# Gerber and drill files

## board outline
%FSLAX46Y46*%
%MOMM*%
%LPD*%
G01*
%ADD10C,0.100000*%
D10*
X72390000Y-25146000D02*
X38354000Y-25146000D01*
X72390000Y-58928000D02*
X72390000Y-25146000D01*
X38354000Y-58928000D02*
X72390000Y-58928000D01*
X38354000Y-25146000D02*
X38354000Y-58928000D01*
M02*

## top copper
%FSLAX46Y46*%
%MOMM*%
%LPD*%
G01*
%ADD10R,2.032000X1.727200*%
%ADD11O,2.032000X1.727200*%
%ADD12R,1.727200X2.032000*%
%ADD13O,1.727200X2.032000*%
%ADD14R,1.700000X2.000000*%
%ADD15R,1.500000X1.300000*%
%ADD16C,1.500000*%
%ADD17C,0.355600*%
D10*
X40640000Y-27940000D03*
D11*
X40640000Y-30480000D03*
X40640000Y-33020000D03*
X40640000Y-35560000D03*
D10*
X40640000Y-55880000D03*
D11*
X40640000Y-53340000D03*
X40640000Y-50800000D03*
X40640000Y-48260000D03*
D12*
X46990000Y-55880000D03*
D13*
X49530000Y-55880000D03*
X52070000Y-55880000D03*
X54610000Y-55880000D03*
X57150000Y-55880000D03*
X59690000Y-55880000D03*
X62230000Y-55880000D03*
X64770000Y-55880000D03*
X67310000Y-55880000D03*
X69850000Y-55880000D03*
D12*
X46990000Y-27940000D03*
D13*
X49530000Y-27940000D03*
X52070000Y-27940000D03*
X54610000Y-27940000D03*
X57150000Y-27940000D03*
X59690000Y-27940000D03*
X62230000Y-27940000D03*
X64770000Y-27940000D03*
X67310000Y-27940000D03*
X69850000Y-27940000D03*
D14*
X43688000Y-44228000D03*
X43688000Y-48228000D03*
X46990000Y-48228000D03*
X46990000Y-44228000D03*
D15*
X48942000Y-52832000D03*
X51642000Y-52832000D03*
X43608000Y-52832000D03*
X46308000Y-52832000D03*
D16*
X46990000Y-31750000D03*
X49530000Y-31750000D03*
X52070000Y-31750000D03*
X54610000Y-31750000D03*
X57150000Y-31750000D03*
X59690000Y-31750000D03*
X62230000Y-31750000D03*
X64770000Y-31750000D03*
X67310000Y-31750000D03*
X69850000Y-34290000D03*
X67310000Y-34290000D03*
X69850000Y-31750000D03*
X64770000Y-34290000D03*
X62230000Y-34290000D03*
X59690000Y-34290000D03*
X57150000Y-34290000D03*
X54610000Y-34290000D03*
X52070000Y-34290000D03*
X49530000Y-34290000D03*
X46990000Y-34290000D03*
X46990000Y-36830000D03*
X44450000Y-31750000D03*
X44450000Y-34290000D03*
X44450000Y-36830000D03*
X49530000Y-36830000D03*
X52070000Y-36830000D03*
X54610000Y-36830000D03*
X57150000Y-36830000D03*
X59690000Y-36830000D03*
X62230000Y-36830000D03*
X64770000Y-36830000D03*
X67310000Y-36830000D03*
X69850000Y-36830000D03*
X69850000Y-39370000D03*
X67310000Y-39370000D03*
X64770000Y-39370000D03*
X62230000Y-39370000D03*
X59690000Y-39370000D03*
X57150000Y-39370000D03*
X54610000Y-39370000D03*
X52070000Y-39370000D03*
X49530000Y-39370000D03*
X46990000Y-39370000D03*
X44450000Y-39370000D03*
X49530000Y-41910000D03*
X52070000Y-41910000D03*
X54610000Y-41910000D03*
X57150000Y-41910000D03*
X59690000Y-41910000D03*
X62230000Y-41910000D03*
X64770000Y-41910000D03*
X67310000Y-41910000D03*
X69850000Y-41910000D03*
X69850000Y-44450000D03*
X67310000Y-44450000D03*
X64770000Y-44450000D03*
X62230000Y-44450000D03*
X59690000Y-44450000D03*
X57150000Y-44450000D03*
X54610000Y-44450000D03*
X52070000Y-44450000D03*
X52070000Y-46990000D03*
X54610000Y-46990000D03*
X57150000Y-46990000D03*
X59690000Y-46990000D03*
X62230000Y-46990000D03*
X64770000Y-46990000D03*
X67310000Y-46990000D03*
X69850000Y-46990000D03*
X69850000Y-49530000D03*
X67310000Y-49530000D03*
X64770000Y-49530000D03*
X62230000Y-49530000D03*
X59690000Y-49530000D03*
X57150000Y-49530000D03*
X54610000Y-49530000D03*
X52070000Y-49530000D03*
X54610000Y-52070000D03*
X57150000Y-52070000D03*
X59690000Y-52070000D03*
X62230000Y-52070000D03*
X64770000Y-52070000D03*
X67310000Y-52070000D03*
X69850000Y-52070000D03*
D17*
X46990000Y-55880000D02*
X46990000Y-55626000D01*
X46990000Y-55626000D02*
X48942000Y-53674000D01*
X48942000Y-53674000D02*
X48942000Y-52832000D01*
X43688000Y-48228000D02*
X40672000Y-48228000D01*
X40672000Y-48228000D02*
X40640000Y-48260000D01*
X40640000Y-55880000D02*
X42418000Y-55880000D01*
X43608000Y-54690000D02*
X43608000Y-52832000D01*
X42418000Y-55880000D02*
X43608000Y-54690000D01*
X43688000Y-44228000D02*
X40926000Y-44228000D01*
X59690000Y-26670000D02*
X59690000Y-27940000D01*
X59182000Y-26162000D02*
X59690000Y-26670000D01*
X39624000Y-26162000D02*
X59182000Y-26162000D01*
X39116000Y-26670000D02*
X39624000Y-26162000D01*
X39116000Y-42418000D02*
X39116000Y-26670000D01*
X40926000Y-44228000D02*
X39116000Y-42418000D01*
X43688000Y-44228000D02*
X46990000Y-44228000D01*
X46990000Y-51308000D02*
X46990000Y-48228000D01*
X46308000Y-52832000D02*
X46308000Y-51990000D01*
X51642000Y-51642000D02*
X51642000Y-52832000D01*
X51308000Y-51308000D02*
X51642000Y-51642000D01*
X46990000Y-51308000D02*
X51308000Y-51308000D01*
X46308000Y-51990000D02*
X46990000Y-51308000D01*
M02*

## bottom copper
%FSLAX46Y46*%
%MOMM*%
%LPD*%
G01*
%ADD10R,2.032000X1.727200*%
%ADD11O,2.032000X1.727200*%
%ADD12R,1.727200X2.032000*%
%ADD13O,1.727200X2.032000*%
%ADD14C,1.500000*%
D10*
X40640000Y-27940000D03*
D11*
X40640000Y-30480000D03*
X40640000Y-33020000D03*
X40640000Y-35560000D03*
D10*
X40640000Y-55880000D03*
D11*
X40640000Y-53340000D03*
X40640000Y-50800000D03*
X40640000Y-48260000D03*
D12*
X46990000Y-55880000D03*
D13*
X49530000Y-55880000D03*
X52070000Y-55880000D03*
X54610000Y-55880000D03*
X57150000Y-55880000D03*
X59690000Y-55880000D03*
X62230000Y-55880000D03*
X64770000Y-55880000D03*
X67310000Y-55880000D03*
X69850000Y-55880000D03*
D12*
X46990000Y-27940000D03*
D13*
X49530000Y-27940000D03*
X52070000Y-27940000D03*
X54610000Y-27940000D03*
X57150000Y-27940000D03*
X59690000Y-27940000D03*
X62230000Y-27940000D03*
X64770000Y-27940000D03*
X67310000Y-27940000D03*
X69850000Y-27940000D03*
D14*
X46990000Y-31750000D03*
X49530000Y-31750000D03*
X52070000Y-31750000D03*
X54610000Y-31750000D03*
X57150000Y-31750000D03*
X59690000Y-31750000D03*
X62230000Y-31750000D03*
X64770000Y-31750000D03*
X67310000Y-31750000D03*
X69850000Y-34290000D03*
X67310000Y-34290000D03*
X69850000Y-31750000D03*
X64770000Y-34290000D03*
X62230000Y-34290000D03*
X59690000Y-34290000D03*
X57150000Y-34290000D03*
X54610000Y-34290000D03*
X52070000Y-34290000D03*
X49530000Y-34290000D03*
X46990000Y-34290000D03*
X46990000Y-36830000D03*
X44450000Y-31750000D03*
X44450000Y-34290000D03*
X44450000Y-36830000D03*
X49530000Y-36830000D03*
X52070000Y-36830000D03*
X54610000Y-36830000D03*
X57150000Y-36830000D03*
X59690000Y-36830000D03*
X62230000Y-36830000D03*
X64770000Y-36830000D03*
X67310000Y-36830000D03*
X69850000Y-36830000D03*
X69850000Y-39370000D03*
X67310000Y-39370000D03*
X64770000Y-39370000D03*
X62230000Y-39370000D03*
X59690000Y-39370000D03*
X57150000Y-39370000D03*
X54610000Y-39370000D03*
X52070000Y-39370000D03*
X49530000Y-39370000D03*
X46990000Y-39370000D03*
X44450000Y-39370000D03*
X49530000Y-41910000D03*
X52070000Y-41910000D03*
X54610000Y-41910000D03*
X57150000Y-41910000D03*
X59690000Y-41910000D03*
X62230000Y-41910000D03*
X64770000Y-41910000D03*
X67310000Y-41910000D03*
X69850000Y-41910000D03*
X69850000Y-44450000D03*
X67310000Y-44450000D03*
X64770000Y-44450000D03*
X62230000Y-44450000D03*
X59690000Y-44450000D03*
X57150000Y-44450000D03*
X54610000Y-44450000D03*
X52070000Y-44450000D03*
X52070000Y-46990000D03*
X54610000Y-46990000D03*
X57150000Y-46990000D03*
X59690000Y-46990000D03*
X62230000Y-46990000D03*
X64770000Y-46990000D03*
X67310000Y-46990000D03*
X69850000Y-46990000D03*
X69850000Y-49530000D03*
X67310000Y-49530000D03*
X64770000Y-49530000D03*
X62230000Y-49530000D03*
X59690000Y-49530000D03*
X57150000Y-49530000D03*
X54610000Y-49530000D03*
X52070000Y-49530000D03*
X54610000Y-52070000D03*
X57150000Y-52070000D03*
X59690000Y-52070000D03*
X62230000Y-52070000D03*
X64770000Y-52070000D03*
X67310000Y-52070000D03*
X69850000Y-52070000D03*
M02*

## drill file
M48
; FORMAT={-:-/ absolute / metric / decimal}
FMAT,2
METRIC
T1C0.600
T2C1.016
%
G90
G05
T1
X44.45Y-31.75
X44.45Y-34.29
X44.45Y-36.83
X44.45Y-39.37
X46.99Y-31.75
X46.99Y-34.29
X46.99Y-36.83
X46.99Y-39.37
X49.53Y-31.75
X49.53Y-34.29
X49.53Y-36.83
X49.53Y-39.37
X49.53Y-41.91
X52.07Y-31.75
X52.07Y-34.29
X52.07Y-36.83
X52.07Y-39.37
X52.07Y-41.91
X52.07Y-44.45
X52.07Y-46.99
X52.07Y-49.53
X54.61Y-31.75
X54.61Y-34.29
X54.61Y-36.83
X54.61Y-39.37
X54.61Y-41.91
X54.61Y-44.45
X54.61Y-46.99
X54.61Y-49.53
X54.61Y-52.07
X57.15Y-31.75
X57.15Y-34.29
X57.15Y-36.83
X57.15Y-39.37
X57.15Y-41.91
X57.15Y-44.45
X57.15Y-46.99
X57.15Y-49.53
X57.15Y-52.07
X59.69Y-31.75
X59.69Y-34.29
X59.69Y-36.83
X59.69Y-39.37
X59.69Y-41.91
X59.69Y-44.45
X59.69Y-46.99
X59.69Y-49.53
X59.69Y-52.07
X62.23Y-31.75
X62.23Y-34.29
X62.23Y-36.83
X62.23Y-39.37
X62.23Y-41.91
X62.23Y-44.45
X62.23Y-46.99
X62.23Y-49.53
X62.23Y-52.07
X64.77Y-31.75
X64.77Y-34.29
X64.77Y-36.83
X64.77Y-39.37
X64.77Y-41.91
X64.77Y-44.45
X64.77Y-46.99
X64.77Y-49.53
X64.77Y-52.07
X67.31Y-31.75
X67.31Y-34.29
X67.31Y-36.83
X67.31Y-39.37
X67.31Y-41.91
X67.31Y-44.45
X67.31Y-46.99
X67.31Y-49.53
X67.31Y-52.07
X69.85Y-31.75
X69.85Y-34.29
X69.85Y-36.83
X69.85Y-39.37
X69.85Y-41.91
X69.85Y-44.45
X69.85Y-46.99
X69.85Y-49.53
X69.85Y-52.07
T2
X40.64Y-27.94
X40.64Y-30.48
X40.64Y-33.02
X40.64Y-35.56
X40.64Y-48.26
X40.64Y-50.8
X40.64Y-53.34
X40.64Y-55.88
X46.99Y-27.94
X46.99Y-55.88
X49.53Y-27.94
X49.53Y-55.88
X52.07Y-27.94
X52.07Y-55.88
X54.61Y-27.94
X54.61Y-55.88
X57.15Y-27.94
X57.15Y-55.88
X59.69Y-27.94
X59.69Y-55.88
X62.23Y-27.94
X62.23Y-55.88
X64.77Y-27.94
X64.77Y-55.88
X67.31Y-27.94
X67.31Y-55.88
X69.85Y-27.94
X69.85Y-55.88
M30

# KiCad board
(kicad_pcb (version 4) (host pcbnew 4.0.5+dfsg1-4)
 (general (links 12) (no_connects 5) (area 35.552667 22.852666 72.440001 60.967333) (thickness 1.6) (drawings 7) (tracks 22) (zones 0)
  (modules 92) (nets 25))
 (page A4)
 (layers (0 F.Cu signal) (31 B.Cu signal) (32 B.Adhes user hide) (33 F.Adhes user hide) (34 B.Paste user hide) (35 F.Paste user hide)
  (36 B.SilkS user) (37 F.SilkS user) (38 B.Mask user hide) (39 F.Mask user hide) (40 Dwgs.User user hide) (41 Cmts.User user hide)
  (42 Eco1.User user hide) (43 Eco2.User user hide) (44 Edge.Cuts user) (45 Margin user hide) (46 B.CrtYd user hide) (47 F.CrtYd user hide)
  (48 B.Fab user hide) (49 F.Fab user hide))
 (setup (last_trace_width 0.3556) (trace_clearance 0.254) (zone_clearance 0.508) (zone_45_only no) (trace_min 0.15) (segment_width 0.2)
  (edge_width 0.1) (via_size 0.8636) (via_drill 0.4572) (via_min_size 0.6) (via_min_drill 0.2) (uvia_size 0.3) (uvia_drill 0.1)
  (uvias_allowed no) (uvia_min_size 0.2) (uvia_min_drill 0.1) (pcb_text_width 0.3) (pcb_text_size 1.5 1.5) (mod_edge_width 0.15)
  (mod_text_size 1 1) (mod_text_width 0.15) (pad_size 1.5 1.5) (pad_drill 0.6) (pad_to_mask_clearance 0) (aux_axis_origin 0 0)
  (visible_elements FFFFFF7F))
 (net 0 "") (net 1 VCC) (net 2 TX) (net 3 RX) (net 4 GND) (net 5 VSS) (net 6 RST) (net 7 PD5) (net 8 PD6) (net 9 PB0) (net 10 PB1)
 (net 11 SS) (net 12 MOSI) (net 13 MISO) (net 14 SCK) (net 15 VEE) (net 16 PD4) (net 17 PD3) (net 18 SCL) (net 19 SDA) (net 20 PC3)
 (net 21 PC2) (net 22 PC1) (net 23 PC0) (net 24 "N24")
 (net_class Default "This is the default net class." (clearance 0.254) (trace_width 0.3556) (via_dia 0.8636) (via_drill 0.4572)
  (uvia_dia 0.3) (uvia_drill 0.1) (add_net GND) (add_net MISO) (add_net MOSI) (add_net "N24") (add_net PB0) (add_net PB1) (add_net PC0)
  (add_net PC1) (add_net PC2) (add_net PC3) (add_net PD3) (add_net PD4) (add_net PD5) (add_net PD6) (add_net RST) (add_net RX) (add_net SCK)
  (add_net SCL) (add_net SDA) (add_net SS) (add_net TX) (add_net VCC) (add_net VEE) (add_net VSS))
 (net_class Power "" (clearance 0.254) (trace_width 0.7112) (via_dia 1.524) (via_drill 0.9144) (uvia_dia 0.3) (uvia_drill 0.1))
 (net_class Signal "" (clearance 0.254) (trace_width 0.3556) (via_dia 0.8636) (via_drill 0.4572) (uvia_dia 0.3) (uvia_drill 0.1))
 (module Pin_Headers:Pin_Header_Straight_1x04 (layer F.Cu) (at 40.64 27.94)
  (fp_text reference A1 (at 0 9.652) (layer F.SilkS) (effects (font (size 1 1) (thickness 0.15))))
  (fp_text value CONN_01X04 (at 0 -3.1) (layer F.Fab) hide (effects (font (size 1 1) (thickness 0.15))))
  (pad 1 thru_hole rect (at 0 0) (size 2.032 1.7272) (drill 1.016) (layers *.Cu *.Mask) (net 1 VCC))
  (pad 2 thru_hole oval (at 0 2.54) (size 2.032 1.7272) (drill 1.016) (layers *.Cu *.Mask) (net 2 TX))
  (pad 3 thru_hole oval (at 0 5.08) (size 2.032 1.7272) (drill 1.016) (layers *.Cu *.Mask) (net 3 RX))
  (pad 4 thru_hole oval (at 0 7.62) (size 2.032 1.7272) (drill 1.016) (layers *.Cu *.Mask) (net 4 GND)))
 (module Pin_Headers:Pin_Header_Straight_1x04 (layer F.Cu) (at 40.64 55.88 180)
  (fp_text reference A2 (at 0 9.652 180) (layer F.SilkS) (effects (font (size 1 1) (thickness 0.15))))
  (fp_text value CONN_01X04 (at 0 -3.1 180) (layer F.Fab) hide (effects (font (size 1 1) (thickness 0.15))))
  (pad 1 thru_hole rect (at 0 0 180) (size 2.032 1.7272) (drill 1.016) (layers *.Cu *.Mask) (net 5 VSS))
  (pad 2 thru_hole oval (at 0 2.54 180) (size 2.032 1.7272) (drill 1.016) (layers *.Cu *.Mask) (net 1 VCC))
  (pad 3 thru_hole oval (at 0 5.08 180) (size 2.032 1.7272) (drill 1.016) (layers *.Cu *.Mask) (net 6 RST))
  (pad 4 thru_hole oval (at 0 7.62 180) (size 2.032 1.7272) (drill 1.016) (layers *.Cu *.Mask) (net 4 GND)))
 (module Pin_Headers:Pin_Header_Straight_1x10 (layer F.Cu) (at 46.99 55.88 90)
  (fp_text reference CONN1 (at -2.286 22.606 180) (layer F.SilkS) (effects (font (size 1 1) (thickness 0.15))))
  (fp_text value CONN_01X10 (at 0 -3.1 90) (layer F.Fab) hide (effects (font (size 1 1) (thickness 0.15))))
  (pad 1 thru_hole rect (at 0 0 90) (size 2.032 1.7272) (drill 1.016) (layers *.Cu *.Mask) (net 1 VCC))
  (pad 2 thru_hole oval (at 0 2.54 90) (size 2.032 1.7272) (drill 1.016) (layers *.Cu *.Mask) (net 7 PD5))
  (pad 3 thru_hole oval (at 0 5.08 90) (size 2.032 1.7272) (drill 1.016) (layers *.Cu *.Mask) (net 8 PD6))
  (pad 4 thru_hole oval (at 0 7.62 90) (size 2.032 1.7272) (drill 1.016) (layers *.Cu *.Mask) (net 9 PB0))
  (pad 5 thru_hole oval (at 0 10.16 90) (size 2.032 1.7272) (drill 1.016) (layers *.Cu *.Mask) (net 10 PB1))
  (pad 6 thru_hole oval (at 0 12.7 90) (size 2.032 1.7272) (drill 1.016) (layers *.Cu *.Mask) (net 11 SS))
  (pad 7 thru_hole oval (at 0 15.24 90) (size 2.032 1.7272) (drill 1.016) (layers *.Cu *.Mask) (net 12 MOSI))
  (pad 8 thru_hole oval (at 0 17.78 90) (size 2.032 1.7272) (drill 1.016) (layers *.Cu *.Mask) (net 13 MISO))
  (pad 9 thru_hole oval (at 0 20.32 90) (size 2.032 1.7272) (drill 1.016) (layers *.Cu *.Mask) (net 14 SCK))
  (pad 10 thru_hole oval (at 0 22.86 90) (size 2.032 1.7272) (drill 1.016) (layers *.Cu *.Mask) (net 4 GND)))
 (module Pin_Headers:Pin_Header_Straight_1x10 (layer F.Cu) (at 46.99 27.94 90)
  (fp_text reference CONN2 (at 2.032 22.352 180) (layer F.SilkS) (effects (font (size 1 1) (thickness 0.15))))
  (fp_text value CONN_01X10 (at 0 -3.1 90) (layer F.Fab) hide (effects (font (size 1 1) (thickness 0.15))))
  (pad 1 thru_hole rect (at 0 0 90) (size 2.032 1.7272) (drill 1.016) (layers *.Cu *.Mask) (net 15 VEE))
  (pad 2 thru_hole oval (at 0 2.54 90) (size 2.032 1.7272) (drill 1.016) (layers *.Cu *.Mask) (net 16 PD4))
  (pad 3 thru_hole oval (at 0 5.08 90) (size 2.032 1.7272) (drill 1.016) (layers *.Cu *.Mask) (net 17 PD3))
  (pad 4 thru_hole oval (at 0 7.62 90) (size 2.032 1.7272) (drill 1.016) (layers *.Cu *.Mask) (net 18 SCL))
  (pad 5 thru_hole oval (at 0 10.16 90) (size 2.032 1.7272) (drill 1.016) (layers *.Cu *.Mask) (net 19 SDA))
  (pad 6 thru_hole oval (at 0 12.7 90) (size 2.032 1.7272) (drill 1.016) (layers *.Cu *.Mask) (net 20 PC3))
  (pad 7 thru_hole oval (at 0 15.24 90) (size 2.032 1.7272) (drill 1.016) (layers *.Cu *.Mask) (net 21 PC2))
  (pad 8 thru_hole oval (at 0 17.78 90) (size 2.032 1.7272) (drill 1.016) (layers *.Cu *.Mask) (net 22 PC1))
  (pad 9 thru_hole oval (at 0 20.32 90) (size 2.032 1.7272) (drill 1.016) (layers *.Cu *.Mask) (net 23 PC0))
  (pad 10 thru_hole oval (at 0 22.86 90) (size 2.032 1.7272) (drill 1.016) (layers *.Cu *.Mask) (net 4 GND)))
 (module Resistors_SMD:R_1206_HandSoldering (layer F.Cu) (at 43.688 46.228 270)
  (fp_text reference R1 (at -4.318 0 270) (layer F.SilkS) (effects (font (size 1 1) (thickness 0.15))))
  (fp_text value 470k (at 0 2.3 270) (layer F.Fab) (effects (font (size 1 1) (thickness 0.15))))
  (pad 1 smd rect (at -2 0 270) (size 2 1.7) (layers F.Cu F.Paste F.Mask) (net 20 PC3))
  (pad 2 smd rect (at 2 0 270) (size 2 1.7) (layers F.Cu F.Paste F.Mask) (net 4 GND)))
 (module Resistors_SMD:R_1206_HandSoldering (layer F.Cu) (at 46.99 46.228 90)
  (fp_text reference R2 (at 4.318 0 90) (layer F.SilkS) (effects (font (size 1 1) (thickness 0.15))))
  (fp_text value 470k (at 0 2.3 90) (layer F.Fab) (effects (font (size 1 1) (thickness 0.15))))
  (pad 1 smd rect (at -2 0 90) (size 2 1.7) (layers F.Cu F.Paste F.Mask) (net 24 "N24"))
  (pad 2 smd rect (at 2 0 90) (size 2 1.7) (layers F.Cu F.Paste F.Mask) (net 20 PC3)))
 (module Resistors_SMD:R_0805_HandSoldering (layer F.Cu) (at 50.292 52.832)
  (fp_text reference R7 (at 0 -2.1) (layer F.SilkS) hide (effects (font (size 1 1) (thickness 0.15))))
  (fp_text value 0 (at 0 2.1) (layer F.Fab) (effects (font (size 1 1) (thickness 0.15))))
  (pad 1 smd rect (at -1.35 0) (size 1.5 1.3) (layers F.Cu F.Paste F.Mask) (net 1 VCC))
  (pad 2 smd rect (at 1.35 0) (size 1.5 1.3) (layers F.Cu F.Paste F.Mask) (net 24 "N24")))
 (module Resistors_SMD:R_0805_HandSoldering (layer F.Cu) (at 44.958 52.832)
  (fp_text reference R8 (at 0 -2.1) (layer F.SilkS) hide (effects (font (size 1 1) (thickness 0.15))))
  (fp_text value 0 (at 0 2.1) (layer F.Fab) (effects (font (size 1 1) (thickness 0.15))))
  (pad 1 smd rect (at -1.35 0) (size 1.5 1.3) (layers F.Cu F.Paste F.Mask) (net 5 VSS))
  (pad 2 smd rect (at 1.35 0) (size 1.5 1.3) (layers F.Cu F.Paste F.Mask) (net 24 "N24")))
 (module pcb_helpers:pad (layer F.Cu) (at 46.99 31.75)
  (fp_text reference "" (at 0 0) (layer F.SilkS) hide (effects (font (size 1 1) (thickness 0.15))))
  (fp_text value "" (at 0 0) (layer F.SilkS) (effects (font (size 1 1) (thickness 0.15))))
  (pad 1 thru_hole circle (at 0 0) (size 1.5 1.5) (drill 0.6) (layers *.Cu *.Mask F.SilkS)))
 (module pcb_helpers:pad (layer F.Cu) (at 49.53 31.75)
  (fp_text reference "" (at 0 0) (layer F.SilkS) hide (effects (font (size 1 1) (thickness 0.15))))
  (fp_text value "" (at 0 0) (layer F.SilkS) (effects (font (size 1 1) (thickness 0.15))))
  (pad 1 thru_hole circle (at 0 0) (size 1.5 1.5) (drill 0.6) (layers *.Cu *.Mask F.SilkS)))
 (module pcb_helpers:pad (layer F.Cu) (at 52.07 31.75)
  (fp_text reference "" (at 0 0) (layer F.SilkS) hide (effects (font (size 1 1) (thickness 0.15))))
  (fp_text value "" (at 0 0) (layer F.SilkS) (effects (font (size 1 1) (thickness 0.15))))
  (pad 1 thru_hole circle (at 0 0) (size 1.5 1.5) (drill 0.6) (layers *.Cu *.Mask F.SilkS)))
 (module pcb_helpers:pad (layer F.Cu) (at 54.61 31.75)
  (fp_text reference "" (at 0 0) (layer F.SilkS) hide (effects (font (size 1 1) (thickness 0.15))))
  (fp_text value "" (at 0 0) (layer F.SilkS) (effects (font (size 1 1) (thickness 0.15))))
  (pad 1 thru_hole circle (at 0 0) (size 1.5 1.5) (drill 0.6) (layers *.Cu *.Mask F.SilkS)))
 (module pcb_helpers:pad (layer F.Cu) (at 57.15 31.75)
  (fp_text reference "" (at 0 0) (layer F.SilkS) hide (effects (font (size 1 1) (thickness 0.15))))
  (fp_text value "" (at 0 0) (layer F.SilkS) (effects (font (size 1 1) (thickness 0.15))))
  (pad 1 thru_hole circle (at 0 0) (size 1.5 1.5) (drill 0.6) (layers *.Cu *.Mask F.SilkS)))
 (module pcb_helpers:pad (layer F.Cu) (at 59.69 31.75)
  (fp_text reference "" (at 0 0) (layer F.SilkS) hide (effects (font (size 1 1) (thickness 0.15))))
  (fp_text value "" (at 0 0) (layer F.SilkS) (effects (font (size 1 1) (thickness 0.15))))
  (pad 1 thru_hole circle (at 0 0) (size 1.5 1.5) (drill 0.6) (layers *.Cu *.Mask F.SilkS)))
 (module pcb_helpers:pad (layer F.Cu) (at 62.23 31.75)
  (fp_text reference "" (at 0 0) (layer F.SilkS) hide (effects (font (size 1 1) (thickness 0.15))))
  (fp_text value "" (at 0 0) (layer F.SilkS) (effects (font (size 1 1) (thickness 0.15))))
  (pad 1 thru_hole circle (at 0 0) (size 1.5 1.5) (drill 0.6) (layers *.Cu *.Mask F.SilkS)))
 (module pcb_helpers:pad (layer F.Cu) (at 64.77 31.75)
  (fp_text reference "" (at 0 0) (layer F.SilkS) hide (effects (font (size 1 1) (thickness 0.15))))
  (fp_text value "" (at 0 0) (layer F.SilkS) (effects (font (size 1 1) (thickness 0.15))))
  (pad 1 thru_hole circle (at 0 0) (size 1.5 1.5) (drill 0.6) (layers *.Cu *.Mask F.SilkS)))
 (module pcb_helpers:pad (layer F.Cu) (at 67.31 31.75)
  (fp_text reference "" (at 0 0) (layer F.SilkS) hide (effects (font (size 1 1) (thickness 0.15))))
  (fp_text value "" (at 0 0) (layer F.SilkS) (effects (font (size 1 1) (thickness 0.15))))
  (pad 1 thru_hole circle (at 0 0) (size 1.5 1.5) (drill 0.6) (layers *.Cu *.Mask F.SilkS)))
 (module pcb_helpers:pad (layer F.Cu) (at 69.85 34.29)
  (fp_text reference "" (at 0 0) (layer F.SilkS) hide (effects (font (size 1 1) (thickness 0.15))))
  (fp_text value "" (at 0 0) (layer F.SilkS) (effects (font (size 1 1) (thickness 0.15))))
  (pad 1 thru_hole circle (at 0 0) (size 1.5 1.5) (drill 0.6) (layers *.Cu *.Mask F.SilkS)))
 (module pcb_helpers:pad (layer F.Cu) (at 67.31 34.29)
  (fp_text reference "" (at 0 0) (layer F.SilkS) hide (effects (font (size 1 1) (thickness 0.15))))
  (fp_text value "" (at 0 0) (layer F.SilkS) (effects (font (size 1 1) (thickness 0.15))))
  (pad 1 thru_hole circle (at 0 0) (size 1.5 1.5) (drill 0.6) (layers *.Cu *.Mask F.SilkS)))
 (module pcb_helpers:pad (layer F.Cu) (at 69.85 31.75)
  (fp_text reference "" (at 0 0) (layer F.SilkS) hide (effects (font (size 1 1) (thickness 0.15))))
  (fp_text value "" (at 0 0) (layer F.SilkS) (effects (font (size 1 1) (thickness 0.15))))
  (pad 1 thru_hole circle (at 0 0) (size 1.5 1.5) (drill 0.6) (layers *.Cu *.Mask F.SilkS)))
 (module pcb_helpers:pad (layer F.Cu) (at 64.77 34.29)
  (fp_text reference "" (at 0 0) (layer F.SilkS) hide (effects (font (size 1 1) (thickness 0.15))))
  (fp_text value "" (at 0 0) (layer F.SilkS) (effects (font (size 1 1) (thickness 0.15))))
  (pad 1 thru_hole circle (at 0 0) (size 1.5 1.5) (drill 0.6) (layers *.Cu *.Mask F.SilkS)))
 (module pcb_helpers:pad (layer F.Cu) (at 62.23 34.29)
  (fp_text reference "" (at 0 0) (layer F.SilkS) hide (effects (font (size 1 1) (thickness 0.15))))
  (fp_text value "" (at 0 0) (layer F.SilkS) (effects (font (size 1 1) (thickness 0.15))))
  (pad 1 thru_hole circle (at 0 0) (size 1.5 1.5) (drill 0.6) (layers *.Cu *.Mask F.SilkS)))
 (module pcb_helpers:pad (layer F.Cu) (at 59.69 34.29)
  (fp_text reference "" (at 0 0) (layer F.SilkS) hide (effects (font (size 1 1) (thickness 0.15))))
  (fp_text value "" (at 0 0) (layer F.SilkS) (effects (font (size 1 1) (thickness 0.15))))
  (pad 1 thru_hole circle (at 0 0) (size 1.5 1.5) (drill 0.6) (layers *.Cu *.Mask F.SilkS)))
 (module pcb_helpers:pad (layer F.Cu) (at 57.15 34.29)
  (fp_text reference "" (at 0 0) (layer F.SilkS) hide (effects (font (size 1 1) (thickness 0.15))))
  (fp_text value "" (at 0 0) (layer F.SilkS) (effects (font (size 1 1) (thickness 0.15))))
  (pad 1 thru_hole circle (at 0 0) (size 1.5 1.5) (drill 0.6) (layers *.Cu *.Mask F.SilkS)))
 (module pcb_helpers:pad (layer F.Cu) (at 54.61 34.29)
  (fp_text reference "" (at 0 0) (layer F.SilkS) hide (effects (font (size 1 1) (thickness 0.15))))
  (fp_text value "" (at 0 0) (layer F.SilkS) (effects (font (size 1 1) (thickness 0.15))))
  (pad 1 thru_hole circle (at 0 0) (size 1.5 1.5) (drill 0.6) (layers *.Cu *.Mask F.SilkS)))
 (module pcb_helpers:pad (layer F.Cu) (at 52.07 34.29)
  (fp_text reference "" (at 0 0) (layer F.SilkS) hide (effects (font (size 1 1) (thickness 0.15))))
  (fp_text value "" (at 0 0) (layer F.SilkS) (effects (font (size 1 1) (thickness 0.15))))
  (pad 1 thru_hole circle (at 0 0) (size 1.5 1.5) (drill 0.6) (layers *.Cu *.Mask F.SilkS)))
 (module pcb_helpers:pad (layer F.Cu) (at 49.53 34.29)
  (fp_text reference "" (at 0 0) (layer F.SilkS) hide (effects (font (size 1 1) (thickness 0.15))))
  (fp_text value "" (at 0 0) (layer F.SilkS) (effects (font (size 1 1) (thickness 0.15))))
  (pad 1 thru_hole circle (at 0 0) (size 1.5 1.5) (drill 0.6) (layers *.Cu *.Mask F.SilkS)))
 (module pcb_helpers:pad (layer F.Cu) (at 46.99 34.29)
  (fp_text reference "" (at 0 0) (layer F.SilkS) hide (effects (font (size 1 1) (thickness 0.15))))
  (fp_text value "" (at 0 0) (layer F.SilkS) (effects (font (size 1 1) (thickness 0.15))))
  (pad 1 thru_hole circle (at 0 0) (size 1.5 1.5) (drill 0.6) (layers *.Cu *.Mask F.SilkS)))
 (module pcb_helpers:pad (layer F.Cu) (at 46.99 36.83)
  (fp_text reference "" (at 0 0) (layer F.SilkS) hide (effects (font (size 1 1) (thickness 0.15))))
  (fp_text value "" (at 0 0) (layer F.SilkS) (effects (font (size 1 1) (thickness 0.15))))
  (pad 1 thru_hole circle (at 0 0) (size 1.5 1.5) (drill 0.6) (layers *.Cu *.Mask F.SilkS)))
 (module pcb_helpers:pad (layer F.Cu) (at 44.45 31.75)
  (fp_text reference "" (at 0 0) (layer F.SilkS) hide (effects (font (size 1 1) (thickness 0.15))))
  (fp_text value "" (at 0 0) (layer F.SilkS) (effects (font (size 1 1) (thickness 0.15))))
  (pad 1 thru_hole circle (at 0 0) (size 1.5 1.5) (drill 0.6) (layers *.Cu *.Mask F.SilkS)))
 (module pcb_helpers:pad (layer F.Cu) (at 44.45 34.29)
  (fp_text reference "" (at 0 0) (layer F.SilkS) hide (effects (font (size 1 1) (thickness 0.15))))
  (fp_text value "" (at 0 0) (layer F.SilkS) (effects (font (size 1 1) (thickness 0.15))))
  (pad 1 thru_hole circle (at 0 0) (size 1.5 1.5) (drill 0.6) (layers *.Cu *.Mask F.SilkS)))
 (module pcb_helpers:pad (layer F.Cu) (at 44.45 36.83)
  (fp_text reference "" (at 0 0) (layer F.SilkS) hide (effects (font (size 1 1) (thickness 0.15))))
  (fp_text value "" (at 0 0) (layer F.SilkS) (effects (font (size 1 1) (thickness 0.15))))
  (pad 1 thru_hole circle (at 0 0) (size 1.5 1.5) (drill 0.6) (layers *.Cu *.Mask F.SilkS)))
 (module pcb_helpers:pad (layer F.Cu) (at 49.53 36.83)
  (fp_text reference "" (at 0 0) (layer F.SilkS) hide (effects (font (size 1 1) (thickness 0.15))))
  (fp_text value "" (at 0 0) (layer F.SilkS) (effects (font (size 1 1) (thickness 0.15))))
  (pad 1 thru_hole circle (at 0 0) (size 1.5 1.5) (drill 0.6) (layers *.Cu *.Mask F.SilkS)))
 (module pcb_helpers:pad (layer F.Cu) (at 52.07 36.83)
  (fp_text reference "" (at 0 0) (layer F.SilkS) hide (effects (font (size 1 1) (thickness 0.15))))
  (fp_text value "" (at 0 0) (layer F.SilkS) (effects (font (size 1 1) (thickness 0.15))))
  (pad 1 thru_hole circle (at 0 0) (size 1.5 1.5) (drill 0.6) (layers *.Cu *.Mask F.SilkS)))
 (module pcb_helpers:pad (layer F.Cu) (at 54.61 36.83)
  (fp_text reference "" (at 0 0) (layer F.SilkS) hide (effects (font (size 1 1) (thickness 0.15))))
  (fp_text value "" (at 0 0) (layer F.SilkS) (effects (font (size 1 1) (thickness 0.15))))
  (pad 1 thru_hole circle (at 0 0) (size 1.5 1.5) (drill 0.6) (layers *.Cu *.Mask F.SilkS)))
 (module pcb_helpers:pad (layer F.Cu) (at 57.15 36.83)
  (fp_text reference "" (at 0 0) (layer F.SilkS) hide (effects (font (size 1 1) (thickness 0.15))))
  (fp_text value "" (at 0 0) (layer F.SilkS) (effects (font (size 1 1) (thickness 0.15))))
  (pad 1 thru_hole circle (at 0 0) (size 1.5 1.5) (drill 0.6) (layers *.Cu *.Mask F.SilkS)))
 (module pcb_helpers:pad (layer F.Cu) (at 59.69 36.83)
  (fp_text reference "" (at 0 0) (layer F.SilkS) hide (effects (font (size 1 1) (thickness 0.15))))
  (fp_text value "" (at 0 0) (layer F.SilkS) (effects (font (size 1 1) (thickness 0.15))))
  (pad 1 thru_hole circle (at 0 0) (size 1.5 1.5) (drill 0.6) (layers *.Cu *.Mask F.SilkS)))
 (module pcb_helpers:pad (layer F.Cu) (at 62.23 36.83)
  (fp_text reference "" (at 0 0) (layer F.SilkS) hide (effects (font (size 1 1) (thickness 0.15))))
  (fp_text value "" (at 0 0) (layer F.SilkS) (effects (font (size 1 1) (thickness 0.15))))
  (pad 1 thru_hole circle (at 0 0) (size 1.5 1.5) (drill 0.6) (layers *.Cu *.Mask F.SilkS)))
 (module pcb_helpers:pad (layer F.Cu) (at 64.77 36.83)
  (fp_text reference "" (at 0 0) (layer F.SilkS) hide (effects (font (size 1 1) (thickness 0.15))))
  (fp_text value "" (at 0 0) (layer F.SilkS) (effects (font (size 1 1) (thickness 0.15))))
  (pad 1 thru_hole circle (at 0 0) (size 1.5 1.5) (drill 0.6) (layers *.Cu *.Mask F.SilkS)))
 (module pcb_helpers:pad (layer F.Cu) (at 67.31 36.83)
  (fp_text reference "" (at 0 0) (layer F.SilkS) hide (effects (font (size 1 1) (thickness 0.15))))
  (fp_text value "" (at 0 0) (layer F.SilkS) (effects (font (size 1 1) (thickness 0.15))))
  (pad 1 thru_hole circle (at 0 0) (size 1.5 1.5) (drill 0.6) (layers *.Cu *.Mask F.SilkS)))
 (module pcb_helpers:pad (layer F.Cu) (at 69.85 36.83)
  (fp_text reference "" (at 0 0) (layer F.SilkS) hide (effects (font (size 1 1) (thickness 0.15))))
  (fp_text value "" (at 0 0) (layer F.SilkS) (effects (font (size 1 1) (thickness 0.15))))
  (pad 1 thru_hole circle (at 0 0) (size 1.5 1.5) (drill 0.6) (layers *.Cu *.Mask F.SilkS)))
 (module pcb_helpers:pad (layer F.Cu) (at 69.85 39.37)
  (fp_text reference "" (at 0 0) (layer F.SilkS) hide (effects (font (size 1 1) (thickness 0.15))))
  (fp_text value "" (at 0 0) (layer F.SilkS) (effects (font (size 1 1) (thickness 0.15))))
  (pad 1 thru_hole circle (at 0 0) (size 1.5 1.5) (drill 0.6) (layers *.Cu *.Mask F.SilkS)))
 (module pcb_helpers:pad (layer F.Cu) (at 67.31 39.37)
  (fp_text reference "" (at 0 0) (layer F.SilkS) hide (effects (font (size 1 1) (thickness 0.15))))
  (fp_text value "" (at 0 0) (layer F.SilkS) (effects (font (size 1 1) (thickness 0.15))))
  (pad 1 thru_hole circle (at 0 0) (size 1.5 1.5) (drill 0.6) (layers *.Cu *.Mask F.SilkS)))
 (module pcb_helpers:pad (layer F.Cu) (at 64.77 39.37)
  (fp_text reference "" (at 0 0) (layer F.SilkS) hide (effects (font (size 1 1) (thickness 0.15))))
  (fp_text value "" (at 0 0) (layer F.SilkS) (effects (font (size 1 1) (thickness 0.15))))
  (pad 1 thru_hole circle (at 0 0) (size 1.5 1.5) (drill 0.6) (layers *.Cu *.Mask F.SilkS)))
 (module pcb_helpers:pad (layer F.Cu) (at 62.23 39.37)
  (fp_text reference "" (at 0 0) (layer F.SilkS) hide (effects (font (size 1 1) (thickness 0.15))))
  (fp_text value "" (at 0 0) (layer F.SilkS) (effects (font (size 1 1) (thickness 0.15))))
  (pad 1 thru_hole circle (at 0 0) (size 1.5 1.5) (drill 0.6) (layers *.Cu *.Mask F.SilkS)))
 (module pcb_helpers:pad (layer F.Cu) (at 59.69 39.37)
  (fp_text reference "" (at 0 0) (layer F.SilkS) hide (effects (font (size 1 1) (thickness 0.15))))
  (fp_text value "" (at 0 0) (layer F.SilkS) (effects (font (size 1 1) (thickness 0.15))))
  (pad 1 thru_hole circle (at 0 0) (size 1.5 1.5) (drill 0.6) (layers *.Cu *.Mask F.SilkS)))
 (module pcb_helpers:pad (layer F.Cu) (at 57.15 39.37)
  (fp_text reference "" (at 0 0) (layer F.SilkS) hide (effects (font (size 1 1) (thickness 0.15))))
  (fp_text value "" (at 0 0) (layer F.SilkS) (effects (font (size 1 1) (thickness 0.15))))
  (pad 1 thru_hole circle (at 0 0) (size 1.5 1.5) (drill 0.6) (layers *.Cu *.Mask F.SilkS)))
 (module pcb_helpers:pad (layer F.Cu) (at 54.61 39.37)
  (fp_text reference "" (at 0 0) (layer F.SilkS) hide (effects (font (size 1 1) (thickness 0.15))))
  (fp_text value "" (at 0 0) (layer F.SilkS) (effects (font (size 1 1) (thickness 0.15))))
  (pad 1 thru_hole circle (at 0 0) (size 1.5 1.5) (drill 0.6) (layers *.Cu *.Mask F.SilkS)))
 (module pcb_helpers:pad (layer F.Cu) (at 52.07 39.37)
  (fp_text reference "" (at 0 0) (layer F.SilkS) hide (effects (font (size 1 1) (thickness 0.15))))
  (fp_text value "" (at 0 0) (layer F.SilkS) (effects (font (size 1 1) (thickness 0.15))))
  (pad 1 thru_hole circle (at 0 0) (size 1.5 1.5) (drill 0.6) (layers *.Cu *.Mask F.SilkS)))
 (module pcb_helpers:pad (layer F.Cu) (at 49.53 39.37)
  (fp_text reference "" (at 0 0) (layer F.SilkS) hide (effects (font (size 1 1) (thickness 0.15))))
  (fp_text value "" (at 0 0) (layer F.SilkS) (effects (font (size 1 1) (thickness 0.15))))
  (pad 1 thru_hole circle (at 0 0) (size 1.5 1.5) (drill 0.6) (layers *.Cu *.Mask F.SilkS)))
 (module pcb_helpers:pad (layer F.Cu) (at 46.99 39.37)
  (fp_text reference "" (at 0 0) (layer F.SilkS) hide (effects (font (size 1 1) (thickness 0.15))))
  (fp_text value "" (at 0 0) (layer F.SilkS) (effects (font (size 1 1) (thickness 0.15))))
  (pad 1 thru_hole circle (at 0 0) (size 1.5 1.5) (drill 0.6) (layers *.Cu *.Mask F.SilkS)))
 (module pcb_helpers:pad (layer F.Cu) (at 44.45 39.37)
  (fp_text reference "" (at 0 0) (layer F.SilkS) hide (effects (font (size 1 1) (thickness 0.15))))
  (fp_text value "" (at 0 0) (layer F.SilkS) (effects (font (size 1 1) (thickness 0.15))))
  (pad 1 thru_hole circle (at 0 0) (size 1.5 1.5) (drill 0.6) (layers *.Cu *.Mask F.SilkS)))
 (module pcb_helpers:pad (layer F.Cu) (at 49.53 41.91)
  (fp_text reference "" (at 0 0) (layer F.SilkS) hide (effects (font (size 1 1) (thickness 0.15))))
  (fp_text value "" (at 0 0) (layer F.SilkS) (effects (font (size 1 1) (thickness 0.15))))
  (pad 1 thru_hole circle (at 0 0) (size 1.5 1.5) (drill 0.6) (layers *.Cu *.Mask F.SilkS)))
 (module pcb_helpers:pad (layer F.Cu) (at 52.07 41.91)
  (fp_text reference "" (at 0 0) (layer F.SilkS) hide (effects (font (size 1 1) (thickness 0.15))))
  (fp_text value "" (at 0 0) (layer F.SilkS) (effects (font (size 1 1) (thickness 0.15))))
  (pad 1 thru_hole circle (at 0 0) (size 1.5 1.5) (drill 0.6) (layers *.Cu *.Mask F.SilkS)))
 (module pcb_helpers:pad (layer F.Cu) (at 54.61 41.91)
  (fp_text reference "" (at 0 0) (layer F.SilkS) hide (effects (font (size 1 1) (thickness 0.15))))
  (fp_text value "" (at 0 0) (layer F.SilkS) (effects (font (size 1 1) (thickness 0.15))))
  (pad 1 thru_hole circle (at 0 0) (size 1.5 1.5) (drill 0.6) (layers *.Cu *.Mask F.SilkS)))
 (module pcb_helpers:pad (layer F.Cu) (at 57.15 41.91)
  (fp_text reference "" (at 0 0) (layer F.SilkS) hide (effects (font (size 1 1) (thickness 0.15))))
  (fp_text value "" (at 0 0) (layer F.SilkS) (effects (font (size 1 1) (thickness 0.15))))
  (pad 1 thru_hole circle (at 0 0) (size 1.5 1.5) (drill 0.6) (layers *.Cu *.Mask F.SilkS)))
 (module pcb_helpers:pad (layer F.Cu) (at 59.69 41.91)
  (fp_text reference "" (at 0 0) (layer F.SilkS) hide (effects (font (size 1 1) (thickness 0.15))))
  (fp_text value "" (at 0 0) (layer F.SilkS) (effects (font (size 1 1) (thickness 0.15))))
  (pad 1 thru_hole circle (at 0 0) (size 1.5 1.5) (drill 0.6) (layers *.Cu *.Mask F.SilkS)))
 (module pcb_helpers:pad (layer F.Cu) (at 62.23 41.91)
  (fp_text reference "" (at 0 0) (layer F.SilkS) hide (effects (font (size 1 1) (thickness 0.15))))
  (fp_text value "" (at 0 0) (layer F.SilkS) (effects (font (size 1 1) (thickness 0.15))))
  (pad 1 thru_hole circle (at 0 0) (size 1.5 1.5) (drill 0.6) (layers *.Cu *.Mask F.SilkS)))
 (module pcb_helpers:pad (layer F.Cu) (at 64.77 41.91)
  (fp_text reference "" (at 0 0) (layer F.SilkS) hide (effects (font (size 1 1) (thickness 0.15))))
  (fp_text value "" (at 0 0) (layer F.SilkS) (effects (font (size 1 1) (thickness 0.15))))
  (pad 1 thru_hole circle (at 0 0) (size 1.5 1.5) (drill 0.6) (layers *.Cu *.Mask F.SilkS)))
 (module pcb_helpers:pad (layer F.Cu) (at 67.31 41.91)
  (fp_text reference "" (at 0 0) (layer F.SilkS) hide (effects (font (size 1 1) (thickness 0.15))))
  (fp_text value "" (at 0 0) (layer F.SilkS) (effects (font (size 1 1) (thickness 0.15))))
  (pad 1 thru_hole circle (at 0 0) (size 1.5 1.5) (drill 0.6) (layers *.Cu *.Mask F.SilkS)))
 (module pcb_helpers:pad (layer F.Cu) (at 69.85 41.91)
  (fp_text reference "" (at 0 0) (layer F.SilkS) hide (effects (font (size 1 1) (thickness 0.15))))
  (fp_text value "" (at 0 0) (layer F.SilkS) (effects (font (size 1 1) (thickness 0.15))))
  (pad 1 thru_hole circle (at 0 0) (size 1.5 1.5) (drill 0.6) (layers *.Cu *.Mask F.SilkS)))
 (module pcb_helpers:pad (layer F.Cu) (at 69.85 44.45)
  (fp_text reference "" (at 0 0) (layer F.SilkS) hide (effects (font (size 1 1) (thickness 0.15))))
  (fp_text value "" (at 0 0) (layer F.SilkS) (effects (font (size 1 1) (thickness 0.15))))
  (pad 1 thru_hole circle (at 0 0) (size 1.5 1.5) (drill 0.6) (layers *.Cu *.Mask F.SilkS)))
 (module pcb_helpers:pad (layer F.Cu) (at 67.31 44.45)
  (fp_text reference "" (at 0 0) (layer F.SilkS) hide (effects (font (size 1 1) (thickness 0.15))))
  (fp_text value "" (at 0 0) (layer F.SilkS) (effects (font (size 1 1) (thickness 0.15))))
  (pad 1 thru_hole circle (at 0 0) (size 1.5 1.5) (drill 0.6) (layers *.Cu *.Mask F.SilkS)))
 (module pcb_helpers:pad (layer F.Cu) (at 64.77 44.45)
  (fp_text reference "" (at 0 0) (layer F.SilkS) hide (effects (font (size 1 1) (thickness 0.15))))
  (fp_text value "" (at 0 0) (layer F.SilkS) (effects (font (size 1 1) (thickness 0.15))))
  (pad 1 thru_hole circle (at 0 0) (size 1.5 1.5) (drill 0.6) (layers *.Cu *.Mask F.SilkS)))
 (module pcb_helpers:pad (layer F.Cu) (at 62.23 44.45)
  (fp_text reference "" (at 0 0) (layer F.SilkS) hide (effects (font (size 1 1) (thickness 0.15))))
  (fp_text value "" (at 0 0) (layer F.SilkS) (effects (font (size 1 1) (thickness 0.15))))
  (pad 1 thru_hole circle (at 0 0) (size 1.5 1.5) (drill 0.6) (layers *.Cu *.Mask F.SilkS)))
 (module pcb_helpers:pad (layer F.Cu) (at 59.69 44.45)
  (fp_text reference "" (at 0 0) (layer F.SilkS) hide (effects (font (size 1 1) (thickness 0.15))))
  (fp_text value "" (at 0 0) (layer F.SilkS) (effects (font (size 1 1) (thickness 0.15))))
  (pad 1 thru_hole circle (at 0 0) (size 1.5 1.5) (drill 0.6) (layers *.Cu *.Mask F.SilkS)))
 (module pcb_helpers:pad (layer F.Cu) (at 57.15 44.45)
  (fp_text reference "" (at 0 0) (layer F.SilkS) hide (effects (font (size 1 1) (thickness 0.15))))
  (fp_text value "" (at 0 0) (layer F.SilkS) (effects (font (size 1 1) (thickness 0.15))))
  (pad 1 thru_hole circle (at 0 0) (size 1.5 1.5) (drill 0.6) (layers *.Cu *.Mask F.SilkS)))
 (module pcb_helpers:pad (layer F.Cu) (at 54.61 44.45)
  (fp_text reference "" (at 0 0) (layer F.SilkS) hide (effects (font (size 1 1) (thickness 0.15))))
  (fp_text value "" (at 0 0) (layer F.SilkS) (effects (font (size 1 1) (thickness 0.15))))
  (pad 1 thru_hole circle (at 0 0) (size 1.5 1.5) (drill 0.6) (layers *.Cu *.Mask F.SilkS)))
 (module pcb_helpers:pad (layer F.Cu) (at 52.07 44.45)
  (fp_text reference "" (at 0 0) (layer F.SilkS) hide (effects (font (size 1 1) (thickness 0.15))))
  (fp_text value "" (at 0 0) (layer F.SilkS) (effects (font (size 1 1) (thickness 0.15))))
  (pad 1 thru_hole circle (at 0 0) (size 1.5 1.5) (drill 0.6) (layers *.Cu *.Mask F.SilkS)))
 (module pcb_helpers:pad (layer F.Cu) (at 52.07 46.99)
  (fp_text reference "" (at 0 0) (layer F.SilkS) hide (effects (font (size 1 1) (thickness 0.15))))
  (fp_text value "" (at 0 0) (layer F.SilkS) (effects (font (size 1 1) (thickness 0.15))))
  (pad 1 thru_hole circle (at 0 0) (size 1.5 1.5) (drill 0.6) (layers *.Cu *.Mask F.SilkS)))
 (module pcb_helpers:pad (layer F.Cu) (at 54.61 46.99)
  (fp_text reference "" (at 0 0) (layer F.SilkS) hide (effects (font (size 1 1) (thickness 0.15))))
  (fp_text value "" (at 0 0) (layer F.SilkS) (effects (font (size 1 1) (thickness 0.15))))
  (pad 1 thru_hole circle (at 0 0) (size 1.5 1.5) (drill 0.6) (layers *.Cu *.Mask F.SilkS)))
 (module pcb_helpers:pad (layer F.Cu) (at 57.15 46.99)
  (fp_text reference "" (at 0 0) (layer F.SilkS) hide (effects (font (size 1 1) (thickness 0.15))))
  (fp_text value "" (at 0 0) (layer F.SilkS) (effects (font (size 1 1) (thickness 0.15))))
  (pad 1 thru_hole circle (at 0 0) (size 1.5 1.5) (drill 0.6) (layers *.Cu *.Mask F.SilkS)))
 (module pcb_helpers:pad (layer F.Cu) (at 59.69 46.99)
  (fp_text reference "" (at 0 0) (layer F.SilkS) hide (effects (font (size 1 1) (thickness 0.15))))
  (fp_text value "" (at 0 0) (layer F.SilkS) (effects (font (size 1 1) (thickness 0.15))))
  (pad 1 thru_hole circle (at 0 0) (size 1.5 1.5) (drill 0.6) (layers *.Cu *.Mask F.SilkS)))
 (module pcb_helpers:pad (layer F.Cu) (at 62.23 46.99)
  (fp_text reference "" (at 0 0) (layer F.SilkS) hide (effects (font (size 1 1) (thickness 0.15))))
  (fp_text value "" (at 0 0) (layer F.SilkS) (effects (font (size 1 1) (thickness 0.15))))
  (pad 1 thru_hole circle (at 0 0) (size 1.5 1.5) (drill 0.6) (layers *.Cu *.Mask F.SilkS)))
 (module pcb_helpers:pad (layer F.Cu) (at 64.77 46.99)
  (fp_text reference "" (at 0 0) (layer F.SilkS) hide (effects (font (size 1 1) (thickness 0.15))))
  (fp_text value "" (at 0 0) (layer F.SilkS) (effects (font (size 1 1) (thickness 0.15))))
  (pad 1 thru_hole circle (at 0 0) (size 1.5 1.5) (drill 0.6) (layers *.Cu *.Mask F.SilkS)))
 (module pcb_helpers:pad (layer F.Cu) (at 67.31 46.99)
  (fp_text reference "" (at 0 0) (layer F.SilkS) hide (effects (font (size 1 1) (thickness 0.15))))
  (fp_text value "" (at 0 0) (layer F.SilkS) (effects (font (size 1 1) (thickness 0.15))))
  (pad 1 thru_hole circle (at 0 0) (size 1.5 1.5) (drill 0.6) (layers *.Cu *.Mask F.SilkS)))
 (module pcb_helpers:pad (layer F.Cu) (at 69.85 46.99)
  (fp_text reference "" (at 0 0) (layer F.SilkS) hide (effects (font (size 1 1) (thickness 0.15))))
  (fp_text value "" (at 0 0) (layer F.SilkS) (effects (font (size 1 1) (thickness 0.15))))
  (pad 1 thru_hole circle (at 0 0) (size 1.5 1.5) (drill 0.6) (layers *.Cu *.Mask F.SilkS)))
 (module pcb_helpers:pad (layer F.Cu) (at 69.85 49.53)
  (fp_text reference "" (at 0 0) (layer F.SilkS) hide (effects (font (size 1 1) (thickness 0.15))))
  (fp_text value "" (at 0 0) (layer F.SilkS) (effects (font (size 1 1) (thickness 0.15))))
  (pad 1 thru_hole circle (at 0 0) (size 1.5 1.5) (drill 0.6) (layers *.Cu *.Mask F.SilkS)))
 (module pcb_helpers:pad (layer F.Cu) (at 67.31 49.53)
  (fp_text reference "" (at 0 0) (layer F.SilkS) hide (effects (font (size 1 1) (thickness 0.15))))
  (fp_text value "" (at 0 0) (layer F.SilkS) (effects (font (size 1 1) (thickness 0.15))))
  (pad 1 thru_hole circle (at 0 0) (size 1.5 1.5) (drill 0.6) (layers *.Cu *.Mask F.SilkS)))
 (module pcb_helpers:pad (layer F.Cu) (at 64.77 49.53)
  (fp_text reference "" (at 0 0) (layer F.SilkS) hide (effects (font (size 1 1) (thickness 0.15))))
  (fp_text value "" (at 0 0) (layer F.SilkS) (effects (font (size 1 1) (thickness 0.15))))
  (pad 1 thru_hole circle (at 0 0) (size 1.5 1.5) (drill 0.6) (layers *.Cu *.Mask F.SilkS)))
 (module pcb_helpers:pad (layer F.Cu) (at 62.23 49.53)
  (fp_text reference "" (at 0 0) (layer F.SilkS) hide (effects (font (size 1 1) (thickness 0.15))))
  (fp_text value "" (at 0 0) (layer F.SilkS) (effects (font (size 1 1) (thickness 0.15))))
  (pad 1 thru_hole circle (at 0 0) (size 1.5 1.5) (drill 0.6) (layers *.Cu *.Mask F.SilkS)))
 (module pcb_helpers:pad (layer F.Cu) (at 59.69 49.53)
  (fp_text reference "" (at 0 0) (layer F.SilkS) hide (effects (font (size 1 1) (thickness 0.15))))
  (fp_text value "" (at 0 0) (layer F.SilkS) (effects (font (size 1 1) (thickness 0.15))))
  (pad 1 thru_hole circle (at 0 0) (size 1.5 1.5) (drill 0.6) (layers *.Cu *.Mask F.SilkS)))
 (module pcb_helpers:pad (layer F.Cu) (at 57.15 49.53)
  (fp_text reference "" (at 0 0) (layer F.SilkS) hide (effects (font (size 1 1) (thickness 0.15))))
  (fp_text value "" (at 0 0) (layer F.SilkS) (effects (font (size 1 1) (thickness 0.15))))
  (pad 1 thru_hole circle (at 0 0) (size 1.5 1.5) (drill 0.6) (layers *.Cu *.Mask F.SilkS)))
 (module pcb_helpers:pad (layer F.Cu) (at 54.61 49.53)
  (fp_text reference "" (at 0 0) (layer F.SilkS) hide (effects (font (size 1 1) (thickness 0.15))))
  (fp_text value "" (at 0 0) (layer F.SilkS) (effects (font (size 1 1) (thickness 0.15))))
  (pad 1 thru_hole circle (at 0 0) (size 1.5 1.5) (drill 0.6) (layers *.Cu *.Mask F.SilkS)))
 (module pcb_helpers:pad (layer F.Cu) (at 52.07 49.53)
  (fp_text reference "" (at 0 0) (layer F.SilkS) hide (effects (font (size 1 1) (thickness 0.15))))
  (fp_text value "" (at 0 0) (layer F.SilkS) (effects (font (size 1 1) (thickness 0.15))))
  (pad 1 thru_hole circle (at 0 0) (size 1.5 1.5) (drill 0.6) (layers *.Cu *.Mask F.SilkS)))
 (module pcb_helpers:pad (layer F.Cu) (at 54.61 52.07)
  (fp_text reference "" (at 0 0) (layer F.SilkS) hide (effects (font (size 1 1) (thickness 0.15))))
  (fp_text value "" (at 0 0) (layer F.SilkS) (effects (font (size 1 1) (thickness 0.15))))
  (pad 1 thru_hole circle (at 0 0) (size 1.5 1.5) (drill 0.6) (layers *.Cu *.Mask F.SilkS)))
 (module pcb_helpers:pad (layer F.Cu) (at 57.15 52.07)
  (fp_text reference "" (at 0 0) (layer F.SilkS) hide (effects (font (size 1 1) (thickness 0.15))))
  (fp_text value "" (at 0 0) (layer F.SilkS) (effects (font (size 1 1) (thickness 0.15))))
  (pad 1 thru_hole circle (at 0 0) (size 1.5 1.5) (drill 0.6) (layers *.Cu *.Mask F.SilkS)))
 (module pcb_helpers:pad (layer F.Cu) (at 59.69 52.07)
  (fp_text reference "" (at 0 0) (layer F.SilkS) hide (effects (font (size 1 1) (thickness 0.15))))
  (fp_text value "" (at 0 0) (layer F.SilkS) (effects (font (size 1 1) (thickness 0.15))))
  (pad 1 thru_hole circle (at 0 0) (size 1.5 1.5) (drill 0.6) (layers *.Cu *.Mask F.SilkS)))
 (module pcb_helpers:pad (layer F.Cu) (at 62.23 52.07)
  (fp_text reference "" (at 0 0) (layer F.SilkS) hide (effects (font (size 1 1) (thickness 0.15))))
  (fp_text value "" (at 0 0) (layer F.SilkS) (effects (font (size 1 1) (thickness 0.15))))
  (pad 1 thru_hole circle (at 0 0) (size 1.5 1.5) (drill 0.6) (layers *.Cu *.Mask F.SilkS)))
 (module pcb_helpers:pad (layer F.Cu) (at 64.77 52.07)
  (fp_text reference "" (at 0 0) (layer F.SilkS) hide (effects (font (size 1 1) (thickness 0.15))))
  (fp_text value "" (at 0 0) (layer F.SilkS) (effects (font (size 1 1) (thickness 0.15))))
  (pad 1 thru_hole circle (at 0 0) (size 1.5 1.5) (drill 0.6) (layers *.Cu *.Mask F.SilkS)))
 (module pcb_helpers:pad (layer F.Cu) (at 67.31 52.07)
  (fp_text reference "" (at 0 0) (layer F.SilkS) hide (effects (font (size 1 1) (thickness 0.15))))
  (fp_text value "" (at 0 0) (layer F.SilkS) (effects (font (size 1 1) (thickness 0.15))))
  (pad 1 thru_hole circle (at 0 0) (size 1.5 1.5) (drill 0.6) (layers *.Cu *.Mask F.SilkS)))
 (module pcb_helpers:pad (layer F.Cu) (at 69.85 52.07)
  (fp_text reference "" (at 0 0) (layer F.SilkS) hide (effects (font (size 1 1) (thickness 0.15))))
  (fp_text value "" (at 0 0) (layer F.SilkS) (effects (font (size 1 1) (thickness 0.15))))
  (pad 1 thru_hole circle (at 0 0) (size 1.5 1.5) (drill 0.6) (layers *.Cu *.Mask F.SilkS)))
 (gr_line (start 72.39 25.146) (end 38.354 25.146) (angle 90) (layer Edge.Cuts) (width 0.1))
 (gr_line (start 72.39 58.928) (end 72.39 25.146) (angle 90) (layer Edge.Cuts) (width 0.1))
 (gr_line (start 38.354 58.928) (end 72.39 58.928) (angle 90) (layer Edge.Cuts) (width 0.1))
 (gr_line (start 38.354 25.146) (end 38.354 58.928) (angle 90) (layer Edge.Cuts) (width 0.1))
 (segment (start 46.99 55.88) (end 46.99 55.626) (width 0.3556) (layer F.Cu) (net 1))
 (segment (start 46.99 55.626) (end 48.942 53.674) (width 0.3556) (layer F.Cu) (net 1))
 (segment (start 48.942 53.674) (end 48.942 52.832) (width 0.3556) (layer F.Cu) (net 1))
 (segment (start 43.688 48.228) (end 40.672 48.228) (width 0.3556) (layer F.Cu) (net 4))
 (segment (start 40.672 48.228) (end 40.64 48.26) (width 0.3556) (layer F.Cu) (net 4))
 (segment (start 40.64 55.88) (end 42.418 55.88) (width 0.3556) (layer F.Cu) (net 5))
 (segment (start 43.608 54.69) (end 43.608 52.832) (width 0.3556) (layer F.Cu) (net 5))
 (segment (start 42.418 55.88) (end 43.608 54.69) (width 0.3556) (layer F.Cu) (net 5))
 (segment (start 43.688 44.228) (end 40.926 44.228) (width 0.3556) (layer F.Cu) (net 20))
 (segment (start 59.69 26.67) (end 59.69 27.94) (width 0.3556) (layer F.Cu) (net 20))
 (segment (start 59.182 26.162) (end 59.69 26.67) (width 0.3556) (layer F.Cu) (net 20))
 (segment (start 39.624 26.162) (end 59.182 26.162) (width 0.3556) (layer F.Cu) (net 20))
 (segment (start 39.116 26.67) (end 39.624 26.162) (width 0.3556) (layer F.Cu) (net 20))
 (segment (start 39.116 42.418) (end 39.116 26.67) (width 0.3556) (layer F.Cu) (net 20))
 (segment (start 40.926 44.228) (end 39.116 42.418) (width 0.3556) (layer F.Cu) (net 20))
 (segment (start 43.688 44.228) (end 46.99 44.228) (width 0.3556) (layer F.Cu) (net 20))
 (segment (start 46.99 51.308) (end 46.99 48.228) (width 0.3556) (layer F.Cu) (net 24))
 (segment (start 46.308 52.832) (end 46.308 51.99) (width 0.3556) (layer F.Cu) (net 24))
 (segment (start 51.642 51.642) (end 51.642 52.832) (width 0.3556) (layer F.Cu) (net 24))
 (segment (start 51.308 51.308) (end 51.642 51.642) (width 0.3556) (layer F.Cu) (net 24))
 (segment (start 46.99 51.308) (end 51.308 51.308) (width 0.3556) (layer F.Cu) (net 24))
 (segment (start 46.308 51.99) (end 46.99 51.308) (width 0.3556) (layer F.Cu) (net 24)))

